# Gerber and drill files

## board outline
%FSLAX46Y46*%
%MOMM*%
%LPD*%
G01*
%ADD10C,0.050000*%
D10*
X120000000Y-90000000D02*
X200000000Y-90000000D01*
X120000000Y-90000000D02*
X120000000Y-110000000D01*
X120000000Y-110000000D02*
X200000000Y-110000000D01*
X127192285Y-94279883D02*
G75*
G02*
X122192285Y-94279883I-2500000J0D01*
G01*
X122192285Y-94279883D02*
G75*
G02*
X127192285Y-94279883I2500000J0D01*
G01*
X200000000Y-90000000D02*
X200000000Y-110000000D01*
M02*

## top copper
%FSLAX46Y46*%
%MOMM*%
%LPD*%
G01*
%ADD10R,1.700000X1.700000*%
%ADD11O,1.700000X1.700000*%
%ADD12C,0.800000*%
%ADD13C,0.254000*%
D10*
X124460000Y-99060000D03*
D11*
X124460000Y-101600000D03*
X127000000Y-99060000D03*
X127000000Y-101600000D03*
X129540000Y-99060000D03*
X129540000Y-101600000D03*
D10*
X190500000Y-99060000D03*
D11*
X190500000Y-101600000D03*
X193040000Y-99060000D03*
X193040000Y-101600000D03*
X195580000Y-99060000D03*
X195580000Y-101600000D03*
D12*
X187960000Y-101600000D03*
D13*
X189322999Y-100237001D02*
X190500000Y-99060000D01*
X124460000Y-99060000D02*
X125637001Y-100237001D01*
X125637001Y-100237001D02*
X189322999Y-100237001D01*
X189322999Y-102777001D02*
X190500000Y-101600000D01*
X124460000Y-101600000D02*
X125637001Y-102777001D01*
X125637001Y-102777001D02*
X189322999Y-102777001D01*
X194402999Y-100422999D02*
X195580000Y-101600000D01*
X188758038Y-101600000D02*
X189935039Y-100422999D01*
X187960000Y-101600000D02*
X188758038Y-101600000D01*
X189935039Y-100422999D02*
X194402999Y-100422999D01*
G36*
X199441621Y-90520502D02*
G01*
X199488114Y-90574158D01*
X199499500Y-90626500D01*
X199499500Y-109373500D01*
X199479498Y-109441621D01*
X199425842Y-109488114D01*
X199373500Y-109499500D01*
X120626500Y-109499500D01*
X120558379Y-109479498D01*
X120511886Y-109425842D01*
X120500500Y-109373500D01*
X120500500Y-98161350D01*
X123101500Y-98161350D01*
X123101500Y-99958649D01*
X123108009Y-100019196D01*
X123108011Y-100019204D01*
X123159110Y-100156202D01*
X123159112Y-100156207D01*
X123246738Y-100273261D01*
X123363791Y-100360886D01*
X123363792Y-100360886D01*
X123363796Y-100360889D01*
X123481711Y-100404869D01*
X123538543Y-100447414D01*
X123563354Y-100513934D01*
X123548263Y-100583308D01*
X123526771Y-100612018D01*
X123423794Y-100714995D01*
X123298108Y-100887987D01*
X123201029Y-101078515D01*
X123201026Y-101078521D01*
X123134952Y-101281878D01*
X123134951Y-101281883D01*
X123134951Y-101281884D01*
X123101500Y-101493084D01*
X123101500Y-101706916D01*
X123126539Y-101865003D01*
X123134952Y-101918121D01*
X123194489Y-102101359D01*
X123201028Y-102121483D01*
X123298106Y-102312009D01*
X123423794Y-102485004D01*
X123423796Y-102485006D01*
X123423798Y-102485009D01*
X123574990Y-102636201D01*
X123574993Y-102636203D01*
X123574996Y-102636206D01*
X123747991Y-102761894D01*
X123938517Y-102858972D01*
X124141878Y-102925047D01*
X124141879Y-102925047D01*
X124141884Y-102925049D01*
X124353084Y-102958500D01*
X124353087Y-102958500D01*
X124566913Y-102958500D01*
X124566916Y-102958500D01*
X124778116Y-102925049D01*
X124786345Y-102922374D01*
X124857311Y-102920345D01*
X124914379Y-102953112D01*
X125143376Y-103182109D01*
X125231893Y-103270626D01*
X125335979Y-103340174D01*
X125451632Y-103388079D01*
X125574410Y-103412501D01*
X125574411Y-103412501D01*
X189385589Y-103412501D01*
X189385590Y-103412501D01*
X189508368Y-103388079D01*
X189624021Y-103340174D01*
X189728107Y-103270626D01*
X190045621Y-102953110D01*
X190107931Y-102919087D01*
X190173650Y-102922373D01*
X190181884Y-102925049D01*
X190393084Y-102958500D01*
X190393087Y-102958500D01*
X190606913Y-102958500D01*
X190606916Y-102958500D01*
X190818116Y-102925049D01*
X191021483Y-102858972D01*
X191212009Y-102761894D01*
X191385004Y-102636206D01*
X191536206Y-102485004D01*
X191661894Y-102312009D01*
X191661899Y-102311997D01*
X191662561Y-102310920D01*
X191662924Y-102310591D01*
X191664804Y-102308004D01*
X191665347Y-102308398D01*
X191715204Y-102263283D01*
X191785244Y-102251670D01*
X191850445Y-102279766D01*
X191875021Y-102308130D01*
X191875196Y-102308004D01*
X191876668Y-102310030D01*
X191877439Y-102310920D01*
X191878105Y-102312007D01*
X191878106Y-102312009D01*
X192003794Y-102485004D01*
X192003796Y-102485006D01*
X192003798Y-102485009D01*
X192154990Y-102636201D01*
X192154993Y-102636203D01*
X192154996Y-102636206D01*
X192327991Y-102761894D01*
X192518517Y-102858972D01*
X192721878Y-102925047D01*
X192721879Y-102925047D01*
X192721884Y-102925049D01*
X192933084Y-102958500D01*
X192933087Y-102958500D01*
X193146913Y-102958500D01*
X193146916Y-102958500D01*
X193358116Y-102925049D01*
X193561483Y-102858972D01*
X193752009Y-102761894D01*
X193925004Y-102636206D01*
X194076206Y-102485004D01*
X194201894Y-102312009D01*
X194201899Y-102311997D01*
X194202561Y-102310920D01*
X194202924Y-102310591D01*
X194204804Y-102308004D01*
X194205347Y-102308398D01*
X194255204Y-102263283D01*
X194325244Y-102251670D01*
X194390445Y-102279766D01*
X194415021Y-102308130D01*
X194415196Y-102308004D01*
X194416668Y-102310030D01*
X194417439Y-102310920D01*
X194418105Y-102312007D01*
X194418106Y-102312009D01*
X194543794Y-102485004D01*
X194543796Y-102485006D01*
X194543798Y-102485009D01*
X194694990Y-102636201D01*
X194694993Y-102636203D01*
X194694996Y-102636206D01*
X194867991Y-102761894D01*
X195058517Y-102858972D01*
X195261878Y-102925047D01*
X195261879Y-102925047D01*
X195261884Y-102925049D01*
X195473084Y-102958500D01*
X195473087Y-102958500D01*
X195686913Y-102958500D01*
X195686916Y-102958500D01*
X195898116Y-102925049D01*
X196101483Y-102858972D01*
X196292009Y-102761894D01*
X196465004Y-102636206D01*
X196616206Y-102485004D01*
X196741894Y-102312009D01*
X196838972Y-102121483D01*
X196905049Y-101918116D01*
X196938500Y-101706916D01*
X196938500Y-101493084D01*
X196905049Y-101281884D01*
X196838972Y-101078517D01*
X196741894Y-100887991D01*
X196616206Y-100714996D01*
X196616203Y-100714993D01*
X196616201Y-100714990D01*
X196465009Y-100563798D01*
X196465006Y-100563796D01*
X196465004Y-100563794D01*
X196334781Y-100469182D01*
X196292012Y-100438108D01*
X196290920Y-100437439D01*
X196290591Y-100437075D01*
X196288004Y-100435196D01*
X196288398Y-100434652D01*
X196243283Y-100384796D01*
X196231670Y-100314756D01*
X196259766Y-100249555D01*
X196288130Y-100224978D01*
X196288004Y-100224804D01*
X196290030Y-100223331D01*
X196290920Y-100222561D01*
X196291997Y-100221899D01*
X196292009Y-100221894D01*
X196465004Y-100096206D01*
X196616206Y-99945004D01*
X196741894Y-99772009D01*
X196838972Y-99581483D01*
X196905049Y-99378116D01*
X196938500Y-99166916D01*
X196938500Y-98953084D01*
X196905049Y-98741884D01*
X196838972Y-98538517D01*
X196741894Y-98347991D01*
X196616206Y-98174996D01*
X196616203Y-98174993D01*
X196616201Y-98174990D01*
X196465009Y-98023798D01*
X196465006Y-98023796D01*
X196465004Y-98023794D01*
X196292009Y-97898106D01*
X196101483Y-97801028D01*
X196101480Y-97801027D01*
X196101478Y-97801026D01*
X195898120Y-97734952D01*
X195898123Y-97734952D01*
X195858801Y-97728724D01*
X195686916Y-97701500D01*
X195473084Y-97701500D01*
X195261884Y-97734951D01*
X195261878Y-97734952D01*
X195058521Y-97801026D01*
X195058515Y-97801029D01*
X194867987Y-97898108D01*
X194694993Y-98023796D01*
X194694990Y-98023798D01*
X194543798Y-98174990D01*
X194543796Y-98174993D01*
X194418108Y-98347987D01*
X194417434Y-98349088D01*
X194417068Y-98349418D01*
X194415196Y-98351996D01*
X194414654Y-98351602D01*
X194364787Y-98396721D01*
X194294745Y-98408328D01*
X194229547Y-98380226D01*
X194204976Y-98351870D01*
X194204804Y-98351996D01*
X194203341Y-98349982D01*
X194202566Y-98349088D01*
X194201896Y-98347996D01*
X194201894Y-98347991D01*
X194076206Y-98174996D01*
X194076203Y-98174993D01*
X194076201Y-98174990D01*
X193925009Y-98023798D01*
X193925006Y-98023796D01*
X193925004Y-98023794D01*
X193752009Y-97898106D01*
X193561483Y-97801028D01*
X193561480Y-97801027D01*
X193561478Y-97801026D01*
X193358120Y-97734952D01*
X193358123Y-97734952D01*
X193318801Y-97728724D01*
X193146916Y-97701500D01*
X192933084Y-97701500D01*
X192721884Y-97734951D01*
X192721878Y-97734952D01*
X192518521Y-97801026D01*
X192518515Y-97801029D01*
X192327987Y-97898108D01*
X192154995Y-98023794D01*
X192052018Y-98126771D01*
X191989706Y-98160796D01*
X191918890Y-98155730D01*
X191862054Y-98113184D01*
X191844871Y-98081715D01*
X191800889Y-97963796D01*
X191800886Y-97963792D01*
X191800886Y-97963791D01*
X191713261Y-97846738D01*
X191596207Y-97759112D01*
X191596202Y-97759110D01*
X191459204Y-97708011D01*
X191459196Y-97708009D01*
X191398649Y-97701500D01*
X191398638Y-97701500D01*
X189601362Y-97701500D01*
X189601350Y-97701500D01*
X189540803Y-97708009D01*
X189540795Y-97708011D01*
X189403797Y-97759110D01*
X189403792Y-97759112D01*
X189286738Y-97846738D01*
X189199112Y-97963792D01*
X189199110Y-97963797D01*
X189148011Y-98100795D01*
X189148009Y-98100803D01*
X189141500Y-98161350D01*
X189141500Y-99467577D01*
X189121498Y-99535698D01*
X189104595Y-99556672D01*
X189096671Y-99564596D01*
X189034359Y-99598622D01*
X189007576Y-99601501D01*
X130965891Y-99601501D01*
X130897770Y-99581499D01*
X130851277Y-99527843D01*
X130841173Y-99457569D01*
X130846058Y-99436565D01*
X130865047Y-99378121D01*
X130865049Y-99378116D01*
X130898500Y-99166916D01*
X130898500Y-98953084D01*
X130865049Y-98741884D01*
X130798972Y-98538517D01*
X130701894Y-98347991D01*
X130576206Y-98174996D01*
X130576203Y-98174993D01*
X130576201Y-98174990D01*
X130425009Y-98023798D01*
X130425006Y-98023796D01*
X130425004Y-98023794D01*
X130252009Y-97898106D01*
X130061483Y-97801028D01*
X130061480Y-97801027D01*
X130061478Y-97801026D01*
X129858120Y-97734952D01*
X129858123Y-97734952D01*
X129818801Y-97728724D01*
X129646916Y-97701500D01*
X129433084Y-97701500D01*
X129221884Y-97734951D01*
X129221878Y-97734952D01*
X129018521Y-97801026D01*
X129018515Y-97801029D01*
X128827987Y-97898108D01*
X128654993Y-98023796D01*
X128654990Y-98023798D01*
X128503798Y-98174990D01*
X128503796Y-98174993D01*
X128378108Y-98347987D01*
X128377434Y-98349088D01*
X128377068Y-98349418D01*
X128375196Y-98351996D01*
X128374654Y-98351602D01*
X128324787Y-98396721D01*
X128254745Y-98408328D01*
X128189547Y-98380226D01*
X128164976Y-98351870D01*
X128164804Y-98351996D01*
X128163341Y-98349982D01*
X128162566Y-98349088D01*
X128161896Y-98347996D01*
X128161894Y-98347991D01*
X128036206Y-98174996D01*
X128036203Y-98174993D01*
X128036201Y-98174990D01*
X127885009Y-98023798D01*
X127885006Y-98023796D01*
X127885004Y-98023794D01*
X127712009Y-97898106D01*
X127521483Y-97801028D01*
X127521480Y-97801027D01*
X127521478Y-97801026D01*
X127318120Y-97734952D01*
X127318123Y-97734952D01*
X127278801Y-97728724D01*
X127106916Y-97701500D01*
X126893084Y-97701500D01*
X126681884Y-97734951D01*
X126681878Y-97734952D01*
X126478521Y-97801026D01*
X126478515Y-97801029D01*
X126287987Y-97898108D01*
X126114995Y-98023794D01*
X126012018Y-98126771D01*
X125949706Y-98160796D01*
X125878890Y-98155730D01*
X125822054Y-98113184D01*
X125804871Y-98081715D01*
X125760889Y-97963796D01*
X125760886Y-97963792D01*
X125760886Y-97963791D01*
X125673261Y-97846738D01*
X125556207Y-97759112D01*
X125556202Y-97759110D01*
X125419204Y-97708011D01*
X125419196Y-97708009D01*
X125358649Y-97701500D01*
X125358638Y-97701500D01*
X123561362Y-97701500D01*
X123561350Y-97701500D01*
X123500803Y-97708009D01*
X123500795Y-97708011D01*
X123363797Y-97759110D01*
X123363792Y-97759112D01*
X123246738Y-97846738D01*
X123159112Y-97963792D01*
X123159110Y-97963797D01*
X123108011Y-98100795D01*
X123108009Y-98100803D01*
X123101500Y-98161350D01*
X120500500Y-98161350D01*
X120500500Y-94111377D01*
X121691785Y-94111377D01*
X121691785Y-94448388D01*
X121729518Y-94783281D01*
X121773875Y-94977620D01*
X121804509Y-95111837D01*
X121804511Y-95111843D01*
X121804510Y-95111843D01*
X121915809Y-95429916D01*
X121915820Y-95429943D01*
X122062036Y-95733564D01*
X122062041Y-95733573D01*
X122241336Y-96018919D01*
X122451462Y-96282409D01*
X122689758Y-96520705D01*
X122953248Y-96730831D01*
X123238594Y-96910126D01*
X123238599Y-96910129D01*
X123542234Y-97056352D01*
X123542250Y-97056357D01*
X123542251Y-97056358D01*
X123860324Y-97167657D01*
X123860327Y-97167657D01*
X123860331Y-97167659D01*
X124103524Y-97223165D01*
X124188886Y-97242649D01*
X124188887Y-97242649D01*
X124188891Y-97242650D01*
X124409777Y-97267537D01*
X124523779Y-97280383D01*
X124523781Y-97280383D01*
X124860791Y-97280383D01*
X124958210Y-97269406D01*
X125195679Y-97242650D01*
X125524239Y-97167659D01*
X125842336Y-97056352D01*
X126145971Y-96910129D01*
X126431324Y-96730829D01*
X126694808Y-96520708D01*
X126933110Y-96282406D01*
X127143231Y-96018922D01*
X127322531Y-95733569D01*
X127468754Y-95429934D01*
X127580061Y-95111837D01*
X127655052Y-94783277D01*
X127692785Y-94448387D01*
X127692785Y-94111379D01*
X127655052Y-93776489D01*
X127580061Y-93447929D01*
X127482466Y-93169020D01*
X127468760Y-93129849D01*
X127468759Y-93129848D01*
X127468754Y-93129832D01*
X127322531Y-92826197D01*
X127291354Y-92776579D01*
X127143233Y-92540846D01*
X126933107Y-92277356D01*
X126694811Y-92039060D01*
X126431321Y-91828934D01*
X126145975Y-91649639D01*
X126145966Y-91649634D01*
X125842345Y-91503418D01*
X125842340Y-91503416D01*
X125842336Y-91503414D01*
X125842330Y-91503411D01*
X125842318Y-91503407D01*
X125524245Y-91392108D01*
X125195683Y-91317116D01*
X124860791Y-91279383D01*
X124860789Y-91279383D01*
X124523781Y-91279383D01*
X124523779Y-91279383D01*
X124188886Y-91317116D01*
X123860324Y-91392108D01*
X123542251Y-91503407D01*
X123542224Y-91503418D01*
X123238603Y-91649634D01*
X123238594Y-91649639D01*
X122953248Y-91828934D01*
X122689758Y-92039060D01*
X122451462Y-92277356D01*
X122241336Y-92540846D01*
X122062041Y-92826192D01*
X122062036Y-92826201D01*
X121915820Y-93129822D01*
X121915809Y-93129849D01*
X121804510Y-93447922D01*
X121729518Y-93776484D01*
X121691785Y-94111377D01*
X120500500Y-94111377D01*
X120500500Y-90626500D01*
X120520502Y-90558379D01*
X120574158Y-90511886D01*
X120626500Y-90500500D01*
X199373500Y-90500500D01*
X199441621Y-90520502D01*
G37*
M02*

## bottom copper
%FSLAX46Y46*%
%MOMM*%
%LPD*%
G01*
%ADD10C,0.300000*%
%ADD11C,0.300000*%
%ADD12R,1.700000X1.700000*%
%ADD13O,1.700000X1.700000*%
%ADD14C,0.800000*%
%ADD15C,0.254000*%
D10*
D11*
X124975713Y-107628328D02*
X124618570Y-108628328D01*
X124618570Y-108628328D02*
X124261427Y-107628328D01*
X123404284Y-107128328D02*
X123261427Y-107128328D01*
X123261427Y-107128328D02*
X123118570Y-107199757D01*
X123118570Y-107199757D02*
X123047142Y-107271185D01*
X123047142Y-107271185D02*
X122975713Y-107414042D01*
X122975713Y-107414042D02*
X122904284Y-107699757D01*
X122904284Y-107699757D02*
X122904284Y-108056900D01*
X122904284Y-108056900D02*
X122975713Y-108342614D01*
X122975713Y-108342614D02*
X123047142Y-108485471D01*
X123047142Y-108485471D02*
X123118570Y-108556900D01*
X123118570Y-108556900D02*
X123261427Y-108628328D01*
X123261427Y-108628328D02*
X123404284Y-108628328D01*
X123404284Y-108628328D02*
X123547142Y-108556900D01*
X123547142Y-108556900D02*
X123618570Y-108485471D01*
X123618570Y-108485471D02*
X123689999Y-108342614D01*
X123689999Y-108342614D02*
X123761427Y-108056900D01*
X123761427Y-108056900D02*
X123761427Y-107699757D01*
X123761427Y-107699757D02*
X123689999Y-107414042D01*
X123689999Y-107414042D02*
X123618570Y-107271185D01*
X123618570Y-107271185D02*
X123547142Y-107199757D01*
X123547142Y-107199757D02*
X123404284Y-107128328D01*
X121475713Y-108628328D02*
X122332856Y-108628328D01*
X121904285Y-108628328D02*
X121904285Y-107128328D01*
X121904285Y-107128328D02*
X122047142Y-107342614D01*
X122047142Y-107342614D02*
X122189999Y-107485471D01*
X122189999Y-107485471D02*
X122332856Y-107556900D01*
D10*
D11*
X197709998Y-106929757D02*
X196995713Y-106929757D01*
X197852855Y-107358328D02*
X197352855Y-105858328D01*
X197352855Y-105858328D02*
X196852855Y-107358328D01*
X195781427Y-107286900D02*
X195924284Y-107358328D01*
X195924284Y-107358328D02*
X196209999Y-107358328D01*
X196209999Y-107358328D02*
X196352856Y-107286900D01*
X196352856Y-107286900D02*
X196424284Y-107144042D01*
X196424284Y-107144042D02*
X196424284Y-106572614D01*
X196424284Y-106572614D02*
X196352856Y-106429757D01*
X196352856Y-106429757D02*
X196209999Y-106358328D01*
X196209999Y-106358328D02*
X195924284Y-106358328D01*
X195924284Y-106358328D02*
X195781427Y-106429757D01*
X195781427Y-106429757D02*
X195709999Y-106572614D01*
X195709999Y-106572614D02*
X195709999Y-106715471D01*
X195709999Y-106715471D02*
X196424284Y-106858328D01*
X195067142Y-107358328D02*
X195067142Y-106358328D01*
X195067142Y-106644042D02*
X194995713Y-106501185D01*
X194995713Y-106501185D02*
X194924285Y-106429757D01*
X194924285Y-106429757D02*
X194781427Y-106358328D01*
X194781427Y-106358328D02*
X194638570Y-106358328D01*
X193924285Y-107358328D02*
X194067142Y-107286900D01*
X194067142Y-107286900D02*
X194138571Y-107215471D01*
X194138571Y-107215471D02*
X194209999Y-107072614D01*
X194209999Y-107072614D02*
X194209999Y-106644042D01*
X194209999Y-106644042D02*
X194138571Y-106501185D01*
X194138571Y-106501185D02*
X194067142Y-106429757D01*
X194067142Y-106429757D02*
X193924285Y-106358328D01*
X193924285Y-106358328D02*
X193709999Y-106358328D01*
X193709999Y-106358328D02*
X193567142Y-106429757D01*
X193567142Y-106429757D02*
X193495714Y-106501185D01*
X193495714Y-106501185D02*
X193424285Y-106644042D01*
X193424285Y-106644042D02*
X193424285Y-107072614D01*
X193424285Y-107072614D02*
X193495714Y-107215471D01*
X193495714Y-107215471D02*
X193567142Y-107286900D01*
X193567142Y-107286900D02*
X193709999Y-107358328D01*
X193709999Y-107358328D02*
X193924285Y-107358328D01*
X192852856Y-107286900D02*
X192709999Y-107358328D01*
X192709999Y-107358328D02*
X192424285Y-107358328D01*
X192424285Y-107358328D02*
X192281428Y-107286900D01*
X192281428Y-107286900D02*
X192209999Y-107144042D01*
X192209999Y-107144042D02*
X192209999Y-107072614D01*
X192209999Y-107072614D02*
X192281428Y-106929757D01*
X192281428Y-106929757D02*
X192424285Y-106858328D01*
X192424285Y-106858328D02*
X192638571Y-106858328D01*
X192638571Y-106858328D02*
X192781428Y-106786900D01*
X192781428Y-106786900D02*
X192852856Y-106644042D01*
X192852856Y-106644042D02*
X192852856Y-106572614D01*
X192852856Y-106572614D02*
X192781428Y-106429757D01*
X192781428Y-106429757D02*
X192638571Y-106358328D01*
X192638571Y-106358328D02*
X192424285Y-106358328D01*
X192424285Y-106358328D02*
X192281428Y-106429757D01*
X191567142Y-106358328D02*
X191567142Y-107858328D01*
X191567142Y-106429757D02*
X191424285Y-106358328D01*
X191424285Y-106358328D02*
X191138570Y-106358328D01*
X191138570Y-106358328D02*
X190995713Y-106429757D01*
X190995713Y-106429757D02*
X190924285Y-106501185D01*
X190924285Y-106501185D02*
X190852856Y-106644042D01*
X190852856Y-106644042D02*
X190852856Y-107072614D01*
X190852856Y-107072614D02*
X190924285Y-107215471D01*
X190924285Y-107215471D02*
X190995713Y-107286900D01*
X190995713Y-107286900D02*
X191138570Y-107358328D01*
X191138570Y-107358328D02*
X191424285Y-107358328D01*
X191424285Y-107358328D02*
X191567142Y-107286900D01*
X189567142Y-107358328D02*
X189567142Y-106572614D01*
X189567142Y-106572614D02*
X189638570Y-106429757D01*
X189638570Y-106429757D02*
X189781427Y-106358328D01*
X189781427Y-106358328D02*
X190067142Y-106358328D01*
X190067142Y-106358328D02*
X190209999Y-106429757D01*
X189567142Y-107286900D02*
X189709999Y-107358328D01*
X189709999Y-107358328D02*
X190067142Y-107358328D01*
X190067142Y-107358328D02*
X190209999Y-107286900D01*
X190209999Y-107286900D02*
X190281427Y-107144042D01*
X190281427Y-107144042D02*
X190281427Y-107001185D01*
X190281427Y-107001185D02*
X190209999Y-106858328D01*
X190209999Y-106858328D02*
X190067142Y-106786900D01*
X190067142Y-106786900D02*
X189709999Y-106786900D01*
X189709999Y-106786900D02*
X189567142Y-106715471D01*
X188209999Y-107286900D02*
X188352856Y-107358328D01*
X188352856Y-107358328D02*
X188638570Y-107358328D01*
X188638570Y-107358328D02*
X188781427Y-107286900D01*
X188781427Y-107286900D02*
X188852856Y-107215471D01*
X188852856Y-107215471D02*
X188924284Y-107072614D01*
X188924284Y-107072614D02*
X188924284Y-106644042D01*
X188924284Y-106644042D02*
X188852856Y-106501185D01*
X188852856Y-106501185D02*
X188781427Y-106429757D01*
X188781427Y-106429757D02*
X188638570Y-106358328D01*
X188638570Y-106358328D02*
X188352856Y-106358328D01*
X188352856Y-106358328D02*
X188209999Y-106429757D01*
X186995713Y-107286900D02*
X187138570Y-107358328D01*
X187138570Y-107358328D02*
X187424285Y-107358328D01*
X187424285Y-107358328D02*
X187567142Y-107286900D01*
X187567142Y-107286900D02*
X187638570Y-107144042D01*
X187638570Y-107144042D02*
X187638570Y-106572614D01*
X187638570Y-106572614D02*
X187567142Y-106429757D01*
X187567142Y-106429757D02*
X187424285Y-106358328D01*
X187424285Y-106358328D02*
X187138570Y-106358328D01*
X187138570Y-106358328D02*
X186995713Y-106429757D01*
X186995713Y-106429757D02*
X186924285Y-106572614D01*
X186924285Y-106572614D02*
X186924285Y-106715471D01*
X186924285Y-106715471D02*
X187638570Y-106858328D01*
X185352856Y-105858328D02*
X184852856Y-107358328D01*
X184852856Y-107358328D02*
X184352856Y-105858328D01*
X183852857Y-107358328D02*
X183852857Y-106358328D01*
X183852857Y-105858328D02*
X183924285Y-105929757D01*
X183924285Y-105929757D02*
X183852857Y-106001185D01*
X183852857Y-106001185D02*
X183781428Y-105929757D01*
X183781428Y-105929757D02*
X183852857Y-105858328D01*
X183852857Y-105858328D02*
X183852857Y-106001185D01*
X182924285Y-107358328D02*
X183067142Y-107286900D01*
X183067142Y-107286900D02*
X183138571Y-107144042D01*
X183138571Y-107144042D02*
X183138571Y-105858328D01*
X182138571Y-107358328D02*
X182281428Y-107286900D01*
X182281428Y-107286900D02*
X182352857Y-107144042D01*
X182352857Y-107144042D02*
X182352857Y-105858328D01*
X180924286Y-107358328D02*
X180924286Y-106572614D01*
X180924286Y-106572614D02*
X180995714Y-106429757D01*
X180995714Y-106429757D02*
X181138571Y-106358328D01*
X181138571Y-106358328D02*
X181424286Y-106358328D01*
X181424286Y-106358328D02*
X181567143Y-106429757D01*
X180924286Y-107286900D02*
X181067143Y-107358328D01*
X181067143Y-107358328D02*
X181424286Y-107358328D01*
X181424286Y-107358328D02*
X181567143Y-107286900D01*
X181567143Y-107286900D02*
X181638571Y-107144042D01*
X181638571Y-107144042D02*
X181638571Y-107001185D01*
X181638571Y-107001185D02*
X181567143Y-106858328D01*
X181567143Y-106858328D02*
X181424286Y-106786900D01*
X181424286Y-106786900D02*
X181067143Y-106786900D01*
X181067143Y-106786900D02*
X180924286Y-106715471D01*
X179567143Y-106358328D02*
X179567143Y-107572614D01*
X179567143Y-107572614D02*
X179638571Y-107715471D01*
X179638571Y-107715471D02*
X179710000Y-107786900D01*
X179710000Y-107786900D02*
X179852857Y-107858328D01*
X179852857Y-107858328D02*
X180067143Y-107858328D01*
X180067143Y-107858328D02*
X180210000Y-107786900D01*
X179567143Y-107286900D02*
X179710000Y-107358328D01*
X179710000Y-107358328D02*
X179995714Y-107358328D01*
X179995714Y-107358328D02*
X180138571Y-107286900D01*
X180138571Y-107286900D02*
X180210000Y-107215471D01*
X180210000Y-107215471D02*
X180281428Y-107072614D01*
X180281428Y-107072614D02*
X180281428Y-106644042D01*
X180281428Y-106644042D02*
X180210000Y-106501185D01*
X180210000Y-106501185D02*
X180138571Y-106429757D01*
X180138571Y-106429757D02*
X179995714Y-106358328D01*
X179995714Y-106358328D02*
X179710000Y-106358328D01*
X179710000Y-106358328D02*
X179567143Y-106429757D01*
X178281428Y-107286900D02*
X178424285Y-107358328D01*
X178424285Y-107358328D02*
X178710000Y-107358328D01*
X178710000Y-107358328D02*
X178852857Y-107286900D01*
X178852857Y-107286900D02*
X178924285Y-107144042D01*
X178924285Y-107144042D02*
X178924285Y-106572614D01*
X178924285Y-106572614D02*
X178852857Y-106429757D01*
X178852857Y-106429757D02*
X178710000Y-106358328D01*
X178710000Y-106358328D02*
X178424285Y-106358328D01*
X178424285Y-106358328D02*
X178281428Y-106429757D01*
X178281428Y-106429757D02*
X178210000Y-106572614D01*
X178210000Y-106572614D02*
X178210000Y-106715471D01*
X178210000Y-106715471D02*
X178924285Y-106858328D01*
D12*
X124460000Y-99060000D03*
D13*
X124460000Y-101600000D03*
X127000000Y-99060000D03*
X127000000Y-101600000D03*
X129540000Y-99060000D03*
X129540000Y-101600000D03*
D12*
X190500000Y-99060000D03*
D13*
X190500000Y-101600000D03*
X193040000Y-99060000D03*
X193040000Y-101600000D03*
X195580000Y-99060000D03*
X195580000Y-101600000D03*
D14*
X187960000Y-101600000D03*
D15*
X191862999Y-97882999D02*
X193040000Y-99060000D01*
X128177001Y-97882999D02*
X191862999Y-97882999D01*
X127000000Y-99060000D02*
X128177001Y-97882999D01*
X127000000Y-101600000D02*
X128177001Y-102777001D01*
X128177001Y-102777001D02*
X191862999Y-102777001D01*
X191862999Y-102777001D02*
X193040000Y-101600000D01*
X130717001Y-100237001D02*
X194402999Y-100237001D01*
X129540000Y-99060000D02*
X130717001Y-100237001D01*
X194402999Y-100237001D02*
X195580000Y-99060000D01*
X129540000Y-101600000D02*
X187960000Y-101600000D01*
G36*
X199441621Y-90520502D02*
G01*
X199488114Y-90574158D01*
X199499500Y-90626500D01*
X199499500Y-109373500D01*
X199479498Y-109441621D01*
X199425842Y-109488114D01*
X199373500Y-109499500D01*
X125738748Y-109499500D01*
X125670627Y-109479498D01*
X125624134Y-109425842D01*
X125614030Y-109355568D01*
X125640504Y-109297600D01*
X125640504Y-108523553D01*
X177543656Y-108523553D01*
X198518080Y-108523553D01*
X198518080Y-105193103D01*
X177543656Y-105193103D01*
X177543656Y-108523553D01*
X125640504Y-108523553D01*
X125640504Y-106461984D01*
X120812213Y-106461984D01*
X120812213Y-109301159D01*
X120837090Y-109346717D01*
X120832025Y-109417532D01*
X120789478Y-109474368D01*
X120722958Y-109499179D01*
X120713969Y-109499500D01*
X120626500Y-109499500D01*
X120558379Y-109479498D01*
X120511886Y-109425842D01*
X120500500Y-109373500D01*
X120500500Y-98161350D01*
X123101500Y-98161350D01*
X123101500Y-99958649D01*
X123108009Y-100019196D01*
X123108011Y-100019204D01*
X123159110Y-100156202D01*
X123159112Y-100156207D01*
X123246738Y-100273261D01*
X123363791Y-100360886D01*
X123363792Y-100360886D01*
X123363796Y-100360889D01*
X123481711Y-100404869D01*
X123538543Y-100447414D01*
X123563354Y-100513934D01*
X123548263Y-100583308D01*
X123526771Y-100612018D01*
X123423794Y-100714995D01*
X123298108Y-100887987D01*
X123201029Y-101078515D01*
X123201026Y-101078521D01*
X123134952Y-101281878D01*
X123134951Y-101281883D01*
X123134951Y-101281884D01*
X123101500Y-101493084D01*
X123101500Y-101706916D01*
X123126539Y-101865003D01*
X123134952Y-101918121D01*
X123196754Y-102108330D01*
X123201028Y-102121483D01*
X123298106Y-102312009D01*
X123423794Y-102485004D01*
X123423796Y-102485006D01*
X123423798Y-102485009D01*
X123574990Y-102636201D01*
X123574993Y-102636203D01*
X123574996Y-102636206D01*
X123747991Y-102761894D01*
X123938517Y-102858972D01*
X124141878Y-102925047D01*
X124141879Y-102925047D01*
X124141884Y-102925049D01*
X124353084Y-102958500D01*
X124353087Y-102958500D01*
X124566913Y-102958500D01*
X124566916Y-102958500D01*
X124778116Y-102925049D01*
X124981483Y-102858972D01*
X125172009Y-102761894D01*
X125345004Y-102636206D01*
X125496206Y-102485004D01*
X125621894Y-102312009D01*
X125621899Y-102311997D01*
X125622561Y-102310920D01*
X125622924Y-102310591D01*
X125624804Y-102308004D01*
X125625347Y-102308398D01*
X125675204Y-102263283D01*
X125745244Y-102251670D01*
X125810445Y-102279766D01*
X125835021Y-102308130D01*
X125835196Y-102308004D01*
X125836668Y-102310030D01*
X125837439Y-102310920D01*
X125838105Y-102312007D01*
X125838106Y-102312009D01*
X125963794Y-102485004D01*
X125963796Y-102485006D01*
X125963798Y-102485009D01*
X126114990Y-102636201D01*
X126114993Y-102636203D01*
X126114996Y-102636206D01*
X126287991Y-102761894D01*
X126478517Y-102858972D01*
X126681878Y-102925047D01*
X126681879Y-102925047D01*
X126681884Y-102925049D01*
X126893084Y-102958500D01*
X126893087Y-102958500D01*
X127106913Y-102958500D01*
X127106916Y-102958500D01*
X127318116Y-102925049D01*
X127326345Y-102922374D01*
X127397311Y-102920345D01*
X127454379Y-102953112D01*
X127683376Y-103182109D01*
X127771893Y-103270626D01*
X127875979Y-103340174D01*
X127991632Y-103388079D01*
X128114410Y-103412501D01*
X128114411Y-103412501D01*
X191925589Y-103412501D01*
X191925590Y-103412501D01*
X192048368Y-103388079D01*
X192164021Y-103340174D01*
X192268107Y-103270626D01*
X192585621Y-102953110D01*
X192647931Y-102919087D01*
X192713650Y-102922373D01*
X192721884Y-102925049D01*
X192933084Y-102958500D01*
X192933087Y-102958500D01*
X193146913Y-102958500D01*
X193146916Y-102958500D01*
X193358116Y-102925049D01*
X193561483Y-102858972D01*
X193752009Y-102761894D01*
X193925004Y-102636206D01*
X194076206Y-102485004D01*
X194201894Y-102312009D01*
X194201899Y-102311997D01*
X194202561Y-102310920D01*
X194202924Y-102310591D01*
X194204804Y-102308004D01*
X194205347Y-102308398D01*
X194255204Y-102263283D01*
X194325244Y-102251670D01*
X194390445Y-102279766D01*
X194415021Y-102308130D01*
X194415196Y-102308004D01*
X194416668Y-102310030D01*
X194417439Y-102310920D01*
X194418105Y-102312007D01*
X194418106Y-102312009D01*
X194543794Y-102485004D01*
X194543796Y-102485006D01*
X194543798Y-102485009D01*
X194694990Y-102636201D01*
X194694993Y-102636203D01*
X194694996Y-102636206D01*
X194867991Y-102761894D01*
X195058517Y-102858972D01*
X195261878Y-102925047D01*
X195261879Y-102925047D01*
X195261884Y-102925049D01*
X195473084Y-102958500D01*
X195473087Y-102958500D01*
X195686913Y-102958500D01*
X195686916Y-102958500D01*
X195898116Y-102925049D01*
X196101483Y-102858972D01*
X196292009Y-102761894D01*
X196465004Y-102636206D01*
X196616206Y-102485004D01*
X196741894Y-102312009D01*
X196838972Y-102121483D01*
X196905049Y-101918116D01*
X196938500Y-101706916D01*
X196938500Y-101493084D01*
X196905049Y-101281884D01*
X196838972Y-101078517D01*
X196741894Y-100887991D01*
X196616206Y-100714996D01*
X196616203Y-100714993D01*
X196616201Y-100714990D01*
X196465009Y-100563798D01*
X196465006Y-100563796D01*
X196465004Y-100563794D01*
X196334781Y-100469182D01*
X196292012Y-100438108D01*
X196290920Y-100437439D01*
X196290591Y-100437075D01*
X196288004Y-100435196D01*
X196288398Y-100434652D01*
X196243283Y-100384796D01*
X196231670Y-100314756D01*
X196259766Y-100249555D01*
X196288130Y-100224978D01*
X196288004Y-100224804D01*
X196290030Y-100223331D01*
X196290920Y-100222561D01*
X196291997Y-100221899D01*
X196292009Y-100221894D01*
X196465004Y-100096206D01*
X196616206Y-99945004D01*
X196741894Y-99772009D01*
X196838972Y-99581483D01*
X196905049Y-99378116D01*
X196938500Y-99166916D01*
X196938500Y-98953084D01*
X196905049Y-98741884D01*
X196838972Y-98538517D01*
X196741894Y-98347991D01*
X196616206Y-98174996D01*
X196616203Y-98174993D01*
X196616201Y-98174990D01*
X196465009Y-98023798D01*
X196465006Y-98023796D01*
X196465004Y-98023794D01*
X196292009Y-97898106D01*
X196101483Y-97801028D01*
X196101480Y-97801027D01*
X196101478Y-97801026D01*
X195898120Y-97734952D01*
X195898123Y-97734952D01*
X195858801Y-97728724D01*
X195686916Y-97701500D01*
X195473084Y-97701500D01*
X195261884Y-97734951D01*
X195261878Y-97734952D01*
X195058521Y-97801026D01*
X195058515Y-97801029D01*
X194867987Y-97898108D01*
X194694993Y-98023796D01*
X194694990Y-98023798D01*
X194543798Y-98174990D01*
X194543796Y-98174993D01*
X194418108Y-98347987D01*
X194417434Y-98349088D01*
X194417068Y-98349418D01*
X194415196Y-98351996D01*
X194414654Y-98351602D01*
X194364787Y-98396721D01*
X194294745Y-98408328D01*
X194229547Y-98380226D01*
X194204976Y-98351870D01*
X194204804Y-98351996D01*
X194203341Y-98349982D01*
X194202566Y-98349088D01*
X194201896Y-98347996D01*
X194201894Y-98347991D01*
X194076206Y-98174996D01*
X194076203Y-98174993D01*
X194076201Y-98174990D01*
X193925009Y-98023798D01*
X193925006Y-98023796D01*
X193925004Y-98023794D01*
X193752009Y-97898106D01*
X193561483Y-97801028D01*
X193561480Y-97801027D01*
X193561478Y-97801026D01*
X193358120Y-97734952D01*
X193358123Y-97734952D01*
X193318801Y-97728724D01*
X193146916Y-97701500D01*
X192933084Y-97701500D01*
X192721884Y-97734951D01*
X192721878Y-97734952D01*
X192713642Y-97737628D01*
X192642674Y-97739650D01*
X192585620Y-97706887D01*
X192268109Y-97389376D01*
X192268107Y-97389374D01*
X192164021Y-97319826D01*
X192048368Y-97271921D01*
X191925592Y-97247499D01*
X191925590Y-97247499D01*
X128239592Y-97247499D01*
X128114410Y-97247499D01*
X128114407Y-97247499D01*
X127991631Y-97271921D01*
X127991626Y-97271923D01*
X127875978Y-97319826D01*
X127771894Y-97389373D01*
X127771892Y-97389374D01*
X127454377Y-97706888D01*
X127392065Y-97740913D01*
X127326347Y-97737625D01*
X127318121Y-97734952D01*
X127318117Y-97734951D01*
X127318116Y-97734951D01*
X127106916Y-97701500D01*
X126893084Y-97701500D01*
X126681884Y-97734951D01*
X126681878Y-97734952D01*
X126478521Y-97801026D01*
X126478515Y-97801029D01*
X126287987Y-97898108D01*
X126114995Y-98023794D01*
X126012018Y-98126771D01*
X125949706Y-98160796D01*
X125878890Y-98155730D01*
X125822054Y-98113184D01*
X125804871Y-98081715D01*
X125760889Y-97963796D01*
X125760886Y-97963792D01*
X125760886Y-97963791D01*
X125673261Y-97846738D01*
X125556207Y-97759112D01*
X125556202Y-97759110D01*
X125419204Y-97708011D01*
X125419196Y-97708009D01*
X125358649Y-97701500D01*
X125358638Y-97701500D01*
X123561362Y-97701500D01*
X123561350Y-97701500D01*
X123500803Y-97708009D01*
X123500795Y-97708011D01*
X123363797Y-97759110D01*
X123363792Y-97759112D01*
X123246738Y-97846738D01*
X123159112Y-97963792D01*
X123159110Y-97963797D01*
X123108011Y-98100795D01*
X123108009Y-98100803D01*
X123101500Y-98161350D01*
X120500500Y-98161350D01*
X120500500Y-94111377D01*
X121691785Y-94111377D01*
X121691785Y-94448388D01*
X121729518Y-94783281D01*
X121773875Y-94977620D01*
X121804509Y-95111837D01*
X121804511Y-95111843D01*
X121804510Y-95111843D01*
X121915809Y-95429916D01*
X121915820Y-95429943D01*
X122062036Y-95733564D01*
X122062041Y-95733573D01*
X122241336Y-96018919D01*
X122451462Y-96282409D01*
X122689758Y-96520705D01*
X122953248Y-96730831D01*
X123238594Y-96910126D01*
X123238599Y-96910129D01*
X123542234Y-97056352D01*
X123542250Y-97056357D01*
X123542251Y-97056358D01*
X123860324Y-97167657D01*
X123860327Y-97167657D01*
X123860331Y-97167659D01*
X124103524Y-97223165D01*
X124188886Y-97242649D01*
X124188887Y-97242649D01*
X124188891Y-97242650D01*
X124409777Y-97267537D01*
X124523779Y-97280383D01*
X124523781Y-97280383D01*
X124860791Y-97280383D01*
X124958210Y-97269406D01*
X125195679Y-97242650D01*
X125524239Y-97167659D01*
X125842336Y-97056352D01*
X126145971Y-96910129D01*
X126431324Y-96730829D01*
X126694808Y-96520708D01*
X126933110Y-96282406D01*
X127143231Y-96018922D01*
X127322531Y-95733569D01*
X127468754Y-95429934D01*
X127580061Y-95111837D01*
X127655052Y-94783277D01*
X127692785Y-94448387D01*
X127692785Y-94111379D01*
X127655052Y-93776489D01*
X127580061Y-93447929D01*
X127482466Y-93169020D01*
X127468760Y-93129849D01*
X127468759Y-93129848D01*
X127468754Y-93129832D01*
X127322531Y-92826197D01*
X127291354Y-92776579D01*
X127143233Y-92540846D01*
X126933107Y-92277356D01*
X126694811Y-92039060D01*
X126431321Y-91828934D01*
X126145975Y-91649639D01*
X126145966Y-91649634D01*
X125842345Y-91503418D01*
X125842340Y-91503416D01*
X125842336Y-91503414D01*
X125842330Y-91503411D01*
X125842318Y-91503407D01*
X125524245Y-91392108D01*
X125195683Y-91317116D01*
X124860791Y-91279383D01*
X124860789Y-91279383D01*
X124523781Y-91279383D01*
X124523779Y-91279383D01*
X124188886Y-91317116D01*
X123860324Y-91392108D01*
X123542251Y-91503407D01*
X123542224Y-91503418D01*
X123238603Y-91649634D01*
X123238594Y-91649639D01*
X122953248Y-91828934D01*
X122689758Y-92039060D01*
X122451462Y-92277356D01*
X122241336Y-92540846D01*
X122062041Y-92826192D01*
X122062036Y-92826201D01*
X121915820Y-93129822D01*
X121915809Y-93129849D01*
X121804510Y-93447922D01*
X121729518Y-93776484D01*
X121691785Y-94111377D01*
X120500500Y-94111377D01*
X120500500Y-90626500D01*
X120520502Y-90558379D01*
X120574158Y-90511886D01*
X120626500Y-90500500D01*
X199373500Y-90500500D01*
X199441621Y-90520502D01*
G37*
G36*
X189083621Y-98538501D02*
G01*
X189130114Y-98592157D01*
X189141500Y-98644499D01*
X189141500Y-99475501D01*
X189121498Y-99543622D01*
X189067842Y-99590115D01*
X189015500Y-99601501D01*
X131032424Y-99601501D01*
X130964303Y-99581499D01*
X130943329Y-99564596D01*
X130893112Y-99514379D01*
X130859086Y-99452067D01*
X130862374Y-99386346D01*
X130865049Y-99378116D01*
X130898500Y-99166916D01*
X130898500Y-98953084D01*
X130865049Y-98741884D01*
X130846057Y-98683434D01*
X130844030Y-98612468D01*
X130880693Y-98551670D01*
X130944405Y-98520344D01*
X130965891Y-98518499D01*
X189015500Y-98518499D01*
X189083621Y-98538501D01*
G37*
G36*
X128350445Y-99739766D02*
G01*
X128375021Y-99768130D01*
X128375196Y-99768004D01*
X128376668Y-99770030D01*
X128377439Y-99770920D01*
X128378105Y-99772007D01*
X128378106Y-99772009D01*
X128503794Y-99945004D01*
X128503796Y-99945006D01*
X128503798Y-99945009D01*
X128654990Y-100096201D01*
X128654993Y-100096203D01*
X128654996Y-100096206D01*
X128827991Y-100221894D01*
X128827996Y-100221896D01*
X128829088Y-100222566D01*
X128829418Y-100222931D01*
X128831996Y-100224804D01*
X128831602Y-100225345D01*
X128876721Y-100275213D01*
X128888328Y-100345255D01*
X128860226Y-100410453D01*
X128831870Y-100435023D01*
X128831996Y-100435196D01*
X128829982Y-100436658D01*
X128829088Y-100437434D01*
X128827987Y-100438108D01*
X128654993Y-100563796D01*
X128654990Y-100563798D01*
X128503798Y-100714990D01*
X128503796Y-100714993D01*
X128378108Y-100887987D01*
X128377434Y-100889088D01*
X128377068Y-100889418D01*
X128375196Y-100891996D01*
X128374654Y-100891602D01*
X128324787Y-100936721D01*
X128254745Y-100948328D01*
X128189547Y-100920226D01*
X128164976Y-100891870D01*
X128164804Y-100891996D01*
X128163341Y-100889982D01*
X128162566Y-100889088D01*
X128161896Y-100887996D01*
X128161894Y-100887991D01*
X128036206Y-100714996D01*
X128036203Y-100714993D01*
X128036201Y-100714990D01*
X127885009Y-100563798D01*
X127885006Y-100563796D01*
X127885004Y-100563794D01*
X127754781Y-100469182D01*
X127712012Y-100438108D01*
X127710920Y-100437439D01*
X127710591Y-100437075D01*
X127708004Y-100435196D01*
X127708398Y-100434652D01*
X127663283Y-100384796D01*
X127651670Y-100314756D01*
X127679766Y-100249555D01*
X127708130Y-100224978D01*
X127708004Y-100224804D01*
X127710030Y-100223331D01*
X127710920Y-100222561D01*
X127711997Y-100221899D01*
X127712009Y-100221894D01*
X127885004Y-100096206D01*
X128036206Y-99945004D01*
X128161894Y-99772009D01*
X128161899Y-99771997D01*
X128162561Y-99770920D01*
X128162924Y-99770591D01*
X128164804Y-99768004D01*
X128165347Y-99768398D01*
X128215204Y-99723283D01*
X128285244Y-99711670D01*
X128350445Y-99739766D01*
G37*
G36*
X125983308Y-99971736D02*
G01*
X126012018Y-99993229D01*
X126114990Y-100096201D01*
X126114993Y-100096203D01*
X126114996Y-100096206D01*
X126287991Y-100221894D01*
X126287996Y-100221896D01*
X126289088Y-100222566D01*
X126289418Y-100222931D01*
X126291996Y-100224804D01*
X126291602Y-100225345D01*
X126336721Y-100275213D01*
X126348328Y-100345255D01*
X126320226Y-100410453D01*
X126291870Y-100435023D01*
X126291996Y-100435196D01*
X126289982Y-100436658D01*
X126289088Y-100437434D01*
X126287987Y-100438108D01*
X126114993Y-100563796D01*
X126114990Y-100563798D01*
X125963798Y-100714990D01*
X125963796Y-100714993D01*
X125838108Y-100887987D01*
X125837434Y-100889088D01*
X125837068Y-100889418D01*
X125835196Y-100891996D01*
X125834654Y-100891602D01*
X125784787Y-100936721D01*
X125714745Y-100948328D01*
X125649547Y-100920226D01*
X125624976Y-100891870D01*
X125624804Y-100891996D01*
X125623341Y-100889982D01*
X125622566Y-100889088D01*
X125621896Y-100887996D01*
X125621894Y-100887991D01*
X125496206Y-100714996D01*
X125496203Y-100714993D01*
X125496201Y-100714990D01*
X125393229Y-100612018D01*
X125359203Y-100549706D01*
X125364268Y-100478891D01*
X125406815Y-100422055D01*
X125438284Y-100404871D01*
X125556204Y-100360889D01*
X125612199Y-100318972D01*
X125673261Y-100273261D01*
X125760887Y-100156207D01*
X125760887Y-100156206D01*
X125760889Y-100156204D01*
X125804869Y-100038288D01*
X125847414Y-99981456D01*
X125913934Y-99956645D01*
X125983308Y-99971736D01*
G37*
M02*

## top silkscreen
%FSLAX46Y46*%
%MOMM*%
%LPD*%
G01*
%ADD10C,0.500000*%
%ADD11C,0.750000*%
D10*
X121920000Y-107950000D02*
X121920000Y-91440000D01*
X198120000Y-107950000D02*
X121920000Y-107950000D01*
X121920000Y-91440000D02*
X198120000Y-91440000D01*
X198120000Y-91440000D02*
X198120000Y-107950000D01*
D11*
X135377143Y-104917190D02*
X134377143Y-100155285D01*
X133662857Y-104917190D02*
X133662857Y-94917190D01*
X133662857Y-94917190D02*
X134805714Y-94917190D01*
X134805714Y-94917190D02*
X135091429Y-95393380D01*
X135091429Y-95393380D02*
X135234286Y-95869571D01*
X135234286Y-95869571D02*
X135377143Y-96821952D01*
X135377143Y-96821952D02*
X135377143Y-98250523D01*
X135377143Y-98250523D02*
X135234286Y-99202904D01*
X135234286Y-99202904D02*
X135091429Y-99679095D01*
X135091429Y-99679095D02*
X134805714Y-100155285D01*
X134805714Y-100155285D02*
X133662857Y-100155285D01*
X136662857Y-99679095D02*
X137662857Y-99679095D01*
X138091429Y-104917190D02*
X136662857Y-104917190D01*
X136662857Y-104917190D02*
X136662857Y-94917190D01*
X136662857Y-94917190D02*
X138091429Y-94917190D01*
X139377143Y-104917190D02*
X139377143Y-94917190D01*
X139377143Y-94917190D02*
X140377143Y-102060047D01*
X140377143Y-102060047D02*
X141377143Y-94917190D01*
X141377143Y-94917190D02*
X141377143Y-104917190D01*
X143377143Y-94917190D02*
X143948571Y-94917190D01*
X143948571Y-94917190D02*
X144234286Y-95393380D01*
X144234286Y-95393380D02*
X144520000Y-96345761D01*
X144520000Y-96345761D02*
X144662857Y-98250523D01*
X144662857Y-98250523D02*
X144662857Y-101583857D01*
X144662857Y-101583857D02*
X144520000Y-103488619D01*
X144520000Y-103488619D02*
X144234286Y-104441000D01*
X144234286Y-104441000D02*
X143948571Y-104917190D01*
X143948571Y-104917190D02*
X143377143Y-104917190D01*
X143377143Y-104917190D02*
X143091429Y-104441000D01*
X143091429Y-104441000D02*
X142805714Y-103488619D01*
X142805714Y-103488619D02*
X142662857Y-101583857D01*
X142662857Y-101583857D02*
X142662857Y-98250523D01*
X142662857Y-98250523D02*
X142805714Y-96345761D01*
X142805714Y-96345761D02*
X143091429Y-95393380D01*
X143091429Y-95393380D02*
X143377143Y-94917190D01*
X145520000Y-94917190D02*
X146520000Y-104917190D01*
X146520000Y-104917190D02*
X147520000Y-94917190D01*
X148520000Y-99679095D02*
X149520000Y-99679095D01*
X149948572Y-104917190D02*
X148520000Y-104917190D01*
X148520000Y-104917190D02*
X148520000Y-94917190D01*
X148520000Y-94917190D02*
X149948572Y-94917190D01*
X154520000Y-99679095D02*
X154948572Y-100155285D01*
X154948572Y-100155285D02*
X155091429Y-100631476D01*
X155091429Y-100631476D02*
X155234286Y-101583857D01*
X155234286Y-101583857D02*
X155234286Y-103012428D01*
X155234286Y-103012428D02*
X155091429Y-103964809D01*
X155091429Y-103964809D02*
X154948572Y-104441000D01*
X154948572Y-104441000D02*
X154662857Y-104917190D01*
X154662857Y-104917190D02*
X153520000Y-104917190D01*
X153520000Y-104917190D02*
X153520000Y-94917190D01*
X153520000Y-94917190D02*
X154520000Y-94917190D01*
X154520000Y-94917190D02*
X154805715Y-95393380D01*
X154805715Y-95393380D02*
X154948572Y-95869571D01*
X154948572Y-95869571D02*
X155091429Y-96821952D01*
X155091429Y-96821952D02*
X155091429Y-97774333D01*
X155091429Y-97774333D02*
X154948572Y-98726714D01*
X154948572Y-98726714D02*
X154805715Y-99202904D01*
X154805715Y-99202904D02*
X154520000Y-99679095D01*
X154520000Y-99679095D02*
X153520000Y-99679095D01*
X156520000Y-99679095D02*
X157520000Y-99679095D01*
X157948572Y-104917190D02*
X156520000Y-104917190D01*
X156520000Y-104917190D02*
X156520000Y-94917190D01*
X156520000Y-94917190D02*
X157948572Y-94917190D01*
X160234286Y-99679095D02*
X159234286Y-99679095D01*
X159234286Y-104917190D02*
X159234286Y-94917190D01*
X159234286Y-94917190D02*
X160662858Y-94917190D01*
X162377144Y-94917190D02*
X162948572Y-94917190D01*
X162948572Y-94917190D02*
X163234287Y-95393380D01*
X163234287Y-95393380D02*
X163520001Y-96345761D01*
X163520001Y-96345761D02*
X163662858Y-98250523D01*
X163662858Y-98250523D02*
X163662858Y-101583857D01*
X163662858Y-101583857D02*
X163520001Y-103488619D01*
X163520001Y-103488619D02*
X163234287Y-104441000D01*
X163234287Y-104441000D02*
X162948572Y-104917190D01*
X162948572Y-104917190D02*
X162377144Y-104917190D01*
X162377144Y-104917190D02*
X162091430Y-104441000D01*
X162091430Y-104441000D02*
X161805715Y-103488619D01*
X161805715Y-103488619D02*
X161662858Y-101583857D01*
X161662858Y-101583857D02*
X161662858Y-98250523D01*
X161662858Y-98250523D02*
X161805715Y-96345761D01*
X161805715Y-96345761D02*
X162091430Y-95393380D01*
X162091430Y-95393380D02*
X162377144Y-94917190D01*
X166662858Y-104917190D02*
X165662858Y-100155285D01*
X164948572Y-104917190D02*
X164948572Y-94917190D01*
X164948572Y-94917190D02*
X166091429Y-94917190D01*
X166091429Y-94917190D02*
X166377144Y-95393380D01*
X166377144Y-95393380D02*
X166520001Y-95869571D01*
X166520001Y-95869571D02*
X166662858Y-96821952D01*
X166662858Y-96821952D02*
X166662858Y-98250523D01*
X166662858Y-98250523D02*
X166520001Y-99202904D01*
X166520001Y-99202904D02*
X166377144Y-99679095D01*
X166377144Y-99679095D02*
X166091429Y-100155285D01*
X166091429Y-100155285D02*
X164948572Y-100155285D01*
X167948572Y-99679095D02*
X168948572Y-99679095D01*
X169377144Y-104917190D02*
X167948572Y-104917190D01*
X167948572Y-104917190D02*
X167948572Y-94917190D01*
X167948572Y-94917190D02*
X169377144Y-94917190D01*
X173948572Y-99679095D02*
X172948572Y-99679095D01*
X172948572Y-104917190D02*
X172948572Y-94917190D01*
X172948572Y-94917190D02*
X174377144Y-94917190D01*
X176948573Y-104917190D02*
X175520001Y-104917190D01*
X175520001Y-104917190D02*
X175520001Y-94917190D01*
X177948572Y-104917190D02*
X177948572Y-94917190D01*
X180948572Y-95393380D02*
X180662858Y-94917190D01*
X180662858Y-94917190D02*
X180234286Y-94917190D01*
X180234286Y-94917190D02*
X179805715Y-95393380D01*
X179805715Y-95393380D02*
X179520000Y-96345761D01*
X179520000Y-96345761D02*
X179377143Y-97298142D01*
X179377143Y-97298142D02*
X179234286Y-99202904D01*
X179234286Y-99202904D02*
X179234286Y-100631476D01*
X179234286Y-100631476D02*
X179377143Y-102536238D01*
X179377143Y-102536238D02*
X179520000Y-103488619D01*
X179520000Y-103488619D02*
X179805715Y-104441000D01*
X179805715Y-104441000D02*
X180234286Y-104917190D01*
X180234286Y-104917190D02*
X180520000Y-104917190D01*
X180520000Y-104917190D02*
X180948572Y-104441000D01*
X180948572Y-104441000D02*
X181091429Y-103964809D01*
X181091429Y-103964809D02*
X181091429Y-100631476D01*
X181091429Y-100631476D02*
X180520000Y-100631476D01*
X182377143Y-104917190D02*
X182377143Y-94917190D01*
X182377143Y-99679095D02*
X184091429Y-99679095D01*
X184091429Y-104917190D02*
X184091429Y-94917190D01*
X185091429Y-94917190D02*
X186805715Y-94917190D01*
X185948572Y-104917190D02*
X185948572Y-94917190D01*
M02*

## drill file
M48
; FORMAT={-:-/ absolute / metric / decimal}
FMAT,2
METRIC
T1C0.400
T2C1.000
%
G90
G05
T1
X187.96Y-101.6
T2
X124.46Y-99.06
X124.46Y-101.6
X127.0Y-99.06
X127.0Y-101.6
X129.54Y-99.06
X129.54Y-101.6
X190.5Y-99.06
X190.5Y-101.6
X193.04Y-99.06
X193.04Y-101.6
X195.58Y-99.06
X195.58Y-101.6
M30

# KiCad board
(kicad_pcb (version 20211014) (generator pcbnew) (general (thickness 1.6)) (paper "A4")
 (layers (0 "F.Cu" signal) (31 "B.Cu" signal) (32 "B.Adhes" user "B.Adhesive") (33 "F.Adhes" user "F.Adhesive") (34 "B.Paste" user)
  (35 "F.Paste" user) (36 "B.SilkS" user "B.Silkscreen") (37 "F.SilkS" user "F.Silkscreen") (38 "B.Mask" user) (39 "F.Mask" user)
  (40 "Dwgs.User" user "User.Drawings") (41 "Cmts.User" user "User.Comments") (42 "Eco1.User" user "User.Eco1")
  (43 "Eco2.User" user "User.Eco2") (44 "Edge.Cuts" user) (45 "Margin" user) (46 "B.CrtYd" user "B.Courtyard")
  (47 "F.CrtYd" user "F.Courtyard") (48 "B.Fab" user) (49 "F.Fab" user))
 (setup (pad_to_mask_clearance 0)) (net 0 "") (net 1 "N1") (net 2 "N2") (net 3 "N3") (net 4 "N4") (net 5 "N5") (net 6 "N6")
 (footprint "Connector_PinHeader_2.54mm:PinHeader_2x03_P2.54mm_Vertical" (layer "B.Cu") (at 124.46 99.06 -90)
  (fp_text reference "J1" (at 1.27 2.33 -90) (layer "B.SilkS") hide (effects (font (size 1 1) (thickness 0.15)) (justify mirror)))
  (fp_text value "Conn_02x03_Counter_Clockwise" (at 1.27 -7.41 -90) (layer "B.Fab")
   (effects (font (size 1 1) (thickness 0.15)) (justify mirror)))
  (pad "1" thru_hole rect locked (at 0 0 270) (size 1.7 1.7) (drill 1) (layers *.Cu *.Mask) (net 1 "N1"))
  (pad "2" thru_hole oval locked (at 2.54 0 270) (size 1.7 1.7) (drill 1) (layers *.Cu *.Mask) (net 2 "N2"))
  (pad "3" thru_hole oval locked (at 0 -2.54 270) (size 1.7 1.7) (drill 1) (layers *.Cu *.Mask) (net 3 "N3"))
  (pad "4" thru_hole oval locked (at 2.54 -2.54 270) (size 1.7 1.7) (drill 1) (layers *.Cu *.Mask) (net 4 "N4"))
  (pad "5" thru_hole oval locked (at 0 -5.08 270) (size 1.7 1.7) (drill 1) (layers *.Cu *.Mask) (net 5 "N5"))
  (pad "6" thru_hole oval locked (at 2.54 -5.08 270) (size 1.7 1.7) (drill 1) (layers *.Cu *.Mask) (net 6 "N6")))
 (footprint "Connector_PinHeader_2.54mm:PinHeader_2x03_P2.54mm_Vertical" (layer "B.Cu") (at 190.5 99.06 -90)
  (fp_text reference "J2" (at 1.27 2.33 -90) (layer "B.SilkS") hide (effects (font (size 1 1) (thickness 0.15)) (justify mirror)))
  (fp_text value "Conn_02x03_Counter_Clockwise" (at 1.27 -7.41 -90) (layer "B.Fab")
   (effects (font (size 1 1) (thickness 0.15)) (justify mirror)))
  (pad "1" thru_hole rect locked (at 0 0 270) (size 1.7 1.7) (drill 1) (layers *.Cu *.Mask) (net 1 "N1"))
  (pad "2" thru_hole oval locked (at 2.54 0 270) (size 1.7 1.7) (drill 1) (layers *.Cu *.Mask) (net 2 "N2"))
  (pad "3" thru_hole oval locked (at 0 -2.54 270) (size 1.7 1.7) (drill 1) (layers *.Cu *.Mask) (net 3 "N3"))
  (pad "4" thru_hole oval locked (at 2.54 -2.54 270) (size 1.7 1.7) (drill 1) (layers *.Cu *.Mask) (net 4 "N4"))
  (pad "5" thru_hole oval locked (at 0 -5.08 270) (size 1.7 1.7) (drill 1) (layers *.Cu *.Mask) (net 5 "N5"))
  (pad "6" thru_hole oval locked (at 2.54 -5.08 270) (size 1.7 1.7) (drill 1) (layers *.Cu *.Mask) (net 6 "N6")))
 (gr_line (start 121.92 107.95) (end 121.92 91.44) (layer "F.SilkS") (width 0.5))
 (gr_line (start 198.12 107.95) (end 121.92 107.95) (layer "F.SilkS") (width 0.5))
 (gr_line (start 121.92 91.44) (end 198.12 91.44) (layer "F.SilkS") (width 0.5))
 (gr_line (start 198.12 91.44) (end 198.12 107.95) (layer "F.SilkS") (width 0.5))
 (gr_line (start 120 90) (end 200 90) (layer "Edge.Cuts") (width 0.05))
 (gr_line (start 120 90) (end 120 110) (layer "Edge.Cuts") (width 0.05))
 (gr_line (start 120 110) (end 200 110) (layer "Edge.Cuts") (width 0.05))
 (gr_circle (center 124.692285 94.279883) (end 127.192285 94.279883) (layer "Edge.Cuts") (width 0.05) (fill none))
 (gr_line (start 200 90) (end 200 110) (layer "Edge.Cuts") (width 0.05))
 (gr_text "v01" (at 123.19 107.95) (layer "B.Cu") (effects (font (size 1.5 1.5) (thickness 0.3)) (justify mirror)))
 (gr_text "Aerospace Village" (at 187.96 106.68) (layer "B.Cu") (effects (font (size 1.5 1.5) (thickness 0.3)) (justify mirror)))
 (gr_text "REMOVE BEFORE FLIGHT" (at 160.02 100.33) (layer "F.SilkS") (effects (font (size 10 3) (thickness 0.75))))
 (segment (start 189.322999 100.237001) (end 190.5 99.06) (width 0.254) (layer "F.Cu") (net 1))
 (segment (start 124.46 99.06) (end 125.637001 100.237001) (width 0.254) (layer "F.Cu") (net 1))
 (segment (start 125.637001 100.237001) (end 189.322999 100.237001) (width 0.254) (layer "F.Cu") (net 1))
 (segment (start 189.322999 102.777001) (end 190.5 101.6) (width 0.254) (layer "F.Cu") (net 2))
 (segment (start 124.46 101.6) (end 125.637001 102.777001) (width 0.254) (layer "F.Cu") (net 2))
 (segment (start 125.637001 102.777001) (end 189.322999 102.777001) (width 0.254) (layer "F.Cu") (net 2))
 (segment (start 191.862999 97.882999) (end 193.04 99.06) (width 0.254) (layer "B.Cu") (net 3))
 (segment (start 128.177001 97.882999) (end 191.862999 97.882999) (width 0.254) (layer "B.Cu") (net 3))
 (segment (start 127 99.06) (end 128.177001 97.882999) (width 0.254) (layer "B.Cu") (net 3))
 (segment (start 127 101.6) (end 128.177001 102.777001) (width 0.254) (layer "B.Cu") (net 4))
 (segment (start 128.177001 102.777001) (end 191.862999 102.777001) (width 0.254) (layer "B.Cu") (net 4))
 (segment (start 191.862999 102.777001) (end 193.04 101.6) (width 0.254) (layer "B.Cu") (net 4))
 (segment (start 130.717001 100.237001) (end 194.402999 100.237001) (width 0.254) (layer "B.Cu") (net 5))
 (segment (start 129.54 99.06) (end 130.717001 100.237001) (width 0.254) (layer "B.Cu") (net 5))
 (segment (start 194.402999 100.237001) (end 195.58 99.06) (width 0.254) (layer "B.Cu") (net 5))
 (segment (start 194.402999 100.422999) (end 195.58 101.6) (width 0.254) (layer "F.Cu") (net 6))
 (segment (start 188.758038 101.6) (end 189.935039 100.422999) (width 0.254) (layer "F.Cu") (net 6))
 (segment (start 187.96 101.6) (end 188.758038 101.6) (width 0.254) (layer "F.Cu") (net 6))
 (segment (start 189.935039 100.422999) (end 194.402999 100.422999) (width 0.254) (layer "F.Cu") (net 6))
 (via (at 187.96 101.6) (size 0.8) (drill 0.4) (layers "F.Cu" "B.Cu") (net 6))
 (segment (start 129.54 101.6) (end 187.96 101.6) (width 0.254) (layer "B.Cu") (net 6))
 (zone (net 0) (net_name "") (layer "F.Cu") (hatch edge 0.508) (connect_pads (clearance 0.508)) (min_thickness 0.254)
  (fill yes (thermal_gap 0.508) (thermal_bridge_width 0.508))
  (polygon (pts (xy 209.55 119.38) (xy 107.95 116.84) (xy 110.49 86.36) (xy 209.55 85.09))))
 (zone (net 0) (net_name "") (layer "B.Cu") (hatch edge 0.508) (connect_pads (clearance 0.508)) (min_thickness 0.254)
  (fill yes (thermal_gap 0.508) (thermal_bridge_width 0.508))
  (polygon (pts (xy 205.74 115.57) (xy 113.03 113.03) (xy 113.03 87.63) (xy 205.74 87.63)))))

